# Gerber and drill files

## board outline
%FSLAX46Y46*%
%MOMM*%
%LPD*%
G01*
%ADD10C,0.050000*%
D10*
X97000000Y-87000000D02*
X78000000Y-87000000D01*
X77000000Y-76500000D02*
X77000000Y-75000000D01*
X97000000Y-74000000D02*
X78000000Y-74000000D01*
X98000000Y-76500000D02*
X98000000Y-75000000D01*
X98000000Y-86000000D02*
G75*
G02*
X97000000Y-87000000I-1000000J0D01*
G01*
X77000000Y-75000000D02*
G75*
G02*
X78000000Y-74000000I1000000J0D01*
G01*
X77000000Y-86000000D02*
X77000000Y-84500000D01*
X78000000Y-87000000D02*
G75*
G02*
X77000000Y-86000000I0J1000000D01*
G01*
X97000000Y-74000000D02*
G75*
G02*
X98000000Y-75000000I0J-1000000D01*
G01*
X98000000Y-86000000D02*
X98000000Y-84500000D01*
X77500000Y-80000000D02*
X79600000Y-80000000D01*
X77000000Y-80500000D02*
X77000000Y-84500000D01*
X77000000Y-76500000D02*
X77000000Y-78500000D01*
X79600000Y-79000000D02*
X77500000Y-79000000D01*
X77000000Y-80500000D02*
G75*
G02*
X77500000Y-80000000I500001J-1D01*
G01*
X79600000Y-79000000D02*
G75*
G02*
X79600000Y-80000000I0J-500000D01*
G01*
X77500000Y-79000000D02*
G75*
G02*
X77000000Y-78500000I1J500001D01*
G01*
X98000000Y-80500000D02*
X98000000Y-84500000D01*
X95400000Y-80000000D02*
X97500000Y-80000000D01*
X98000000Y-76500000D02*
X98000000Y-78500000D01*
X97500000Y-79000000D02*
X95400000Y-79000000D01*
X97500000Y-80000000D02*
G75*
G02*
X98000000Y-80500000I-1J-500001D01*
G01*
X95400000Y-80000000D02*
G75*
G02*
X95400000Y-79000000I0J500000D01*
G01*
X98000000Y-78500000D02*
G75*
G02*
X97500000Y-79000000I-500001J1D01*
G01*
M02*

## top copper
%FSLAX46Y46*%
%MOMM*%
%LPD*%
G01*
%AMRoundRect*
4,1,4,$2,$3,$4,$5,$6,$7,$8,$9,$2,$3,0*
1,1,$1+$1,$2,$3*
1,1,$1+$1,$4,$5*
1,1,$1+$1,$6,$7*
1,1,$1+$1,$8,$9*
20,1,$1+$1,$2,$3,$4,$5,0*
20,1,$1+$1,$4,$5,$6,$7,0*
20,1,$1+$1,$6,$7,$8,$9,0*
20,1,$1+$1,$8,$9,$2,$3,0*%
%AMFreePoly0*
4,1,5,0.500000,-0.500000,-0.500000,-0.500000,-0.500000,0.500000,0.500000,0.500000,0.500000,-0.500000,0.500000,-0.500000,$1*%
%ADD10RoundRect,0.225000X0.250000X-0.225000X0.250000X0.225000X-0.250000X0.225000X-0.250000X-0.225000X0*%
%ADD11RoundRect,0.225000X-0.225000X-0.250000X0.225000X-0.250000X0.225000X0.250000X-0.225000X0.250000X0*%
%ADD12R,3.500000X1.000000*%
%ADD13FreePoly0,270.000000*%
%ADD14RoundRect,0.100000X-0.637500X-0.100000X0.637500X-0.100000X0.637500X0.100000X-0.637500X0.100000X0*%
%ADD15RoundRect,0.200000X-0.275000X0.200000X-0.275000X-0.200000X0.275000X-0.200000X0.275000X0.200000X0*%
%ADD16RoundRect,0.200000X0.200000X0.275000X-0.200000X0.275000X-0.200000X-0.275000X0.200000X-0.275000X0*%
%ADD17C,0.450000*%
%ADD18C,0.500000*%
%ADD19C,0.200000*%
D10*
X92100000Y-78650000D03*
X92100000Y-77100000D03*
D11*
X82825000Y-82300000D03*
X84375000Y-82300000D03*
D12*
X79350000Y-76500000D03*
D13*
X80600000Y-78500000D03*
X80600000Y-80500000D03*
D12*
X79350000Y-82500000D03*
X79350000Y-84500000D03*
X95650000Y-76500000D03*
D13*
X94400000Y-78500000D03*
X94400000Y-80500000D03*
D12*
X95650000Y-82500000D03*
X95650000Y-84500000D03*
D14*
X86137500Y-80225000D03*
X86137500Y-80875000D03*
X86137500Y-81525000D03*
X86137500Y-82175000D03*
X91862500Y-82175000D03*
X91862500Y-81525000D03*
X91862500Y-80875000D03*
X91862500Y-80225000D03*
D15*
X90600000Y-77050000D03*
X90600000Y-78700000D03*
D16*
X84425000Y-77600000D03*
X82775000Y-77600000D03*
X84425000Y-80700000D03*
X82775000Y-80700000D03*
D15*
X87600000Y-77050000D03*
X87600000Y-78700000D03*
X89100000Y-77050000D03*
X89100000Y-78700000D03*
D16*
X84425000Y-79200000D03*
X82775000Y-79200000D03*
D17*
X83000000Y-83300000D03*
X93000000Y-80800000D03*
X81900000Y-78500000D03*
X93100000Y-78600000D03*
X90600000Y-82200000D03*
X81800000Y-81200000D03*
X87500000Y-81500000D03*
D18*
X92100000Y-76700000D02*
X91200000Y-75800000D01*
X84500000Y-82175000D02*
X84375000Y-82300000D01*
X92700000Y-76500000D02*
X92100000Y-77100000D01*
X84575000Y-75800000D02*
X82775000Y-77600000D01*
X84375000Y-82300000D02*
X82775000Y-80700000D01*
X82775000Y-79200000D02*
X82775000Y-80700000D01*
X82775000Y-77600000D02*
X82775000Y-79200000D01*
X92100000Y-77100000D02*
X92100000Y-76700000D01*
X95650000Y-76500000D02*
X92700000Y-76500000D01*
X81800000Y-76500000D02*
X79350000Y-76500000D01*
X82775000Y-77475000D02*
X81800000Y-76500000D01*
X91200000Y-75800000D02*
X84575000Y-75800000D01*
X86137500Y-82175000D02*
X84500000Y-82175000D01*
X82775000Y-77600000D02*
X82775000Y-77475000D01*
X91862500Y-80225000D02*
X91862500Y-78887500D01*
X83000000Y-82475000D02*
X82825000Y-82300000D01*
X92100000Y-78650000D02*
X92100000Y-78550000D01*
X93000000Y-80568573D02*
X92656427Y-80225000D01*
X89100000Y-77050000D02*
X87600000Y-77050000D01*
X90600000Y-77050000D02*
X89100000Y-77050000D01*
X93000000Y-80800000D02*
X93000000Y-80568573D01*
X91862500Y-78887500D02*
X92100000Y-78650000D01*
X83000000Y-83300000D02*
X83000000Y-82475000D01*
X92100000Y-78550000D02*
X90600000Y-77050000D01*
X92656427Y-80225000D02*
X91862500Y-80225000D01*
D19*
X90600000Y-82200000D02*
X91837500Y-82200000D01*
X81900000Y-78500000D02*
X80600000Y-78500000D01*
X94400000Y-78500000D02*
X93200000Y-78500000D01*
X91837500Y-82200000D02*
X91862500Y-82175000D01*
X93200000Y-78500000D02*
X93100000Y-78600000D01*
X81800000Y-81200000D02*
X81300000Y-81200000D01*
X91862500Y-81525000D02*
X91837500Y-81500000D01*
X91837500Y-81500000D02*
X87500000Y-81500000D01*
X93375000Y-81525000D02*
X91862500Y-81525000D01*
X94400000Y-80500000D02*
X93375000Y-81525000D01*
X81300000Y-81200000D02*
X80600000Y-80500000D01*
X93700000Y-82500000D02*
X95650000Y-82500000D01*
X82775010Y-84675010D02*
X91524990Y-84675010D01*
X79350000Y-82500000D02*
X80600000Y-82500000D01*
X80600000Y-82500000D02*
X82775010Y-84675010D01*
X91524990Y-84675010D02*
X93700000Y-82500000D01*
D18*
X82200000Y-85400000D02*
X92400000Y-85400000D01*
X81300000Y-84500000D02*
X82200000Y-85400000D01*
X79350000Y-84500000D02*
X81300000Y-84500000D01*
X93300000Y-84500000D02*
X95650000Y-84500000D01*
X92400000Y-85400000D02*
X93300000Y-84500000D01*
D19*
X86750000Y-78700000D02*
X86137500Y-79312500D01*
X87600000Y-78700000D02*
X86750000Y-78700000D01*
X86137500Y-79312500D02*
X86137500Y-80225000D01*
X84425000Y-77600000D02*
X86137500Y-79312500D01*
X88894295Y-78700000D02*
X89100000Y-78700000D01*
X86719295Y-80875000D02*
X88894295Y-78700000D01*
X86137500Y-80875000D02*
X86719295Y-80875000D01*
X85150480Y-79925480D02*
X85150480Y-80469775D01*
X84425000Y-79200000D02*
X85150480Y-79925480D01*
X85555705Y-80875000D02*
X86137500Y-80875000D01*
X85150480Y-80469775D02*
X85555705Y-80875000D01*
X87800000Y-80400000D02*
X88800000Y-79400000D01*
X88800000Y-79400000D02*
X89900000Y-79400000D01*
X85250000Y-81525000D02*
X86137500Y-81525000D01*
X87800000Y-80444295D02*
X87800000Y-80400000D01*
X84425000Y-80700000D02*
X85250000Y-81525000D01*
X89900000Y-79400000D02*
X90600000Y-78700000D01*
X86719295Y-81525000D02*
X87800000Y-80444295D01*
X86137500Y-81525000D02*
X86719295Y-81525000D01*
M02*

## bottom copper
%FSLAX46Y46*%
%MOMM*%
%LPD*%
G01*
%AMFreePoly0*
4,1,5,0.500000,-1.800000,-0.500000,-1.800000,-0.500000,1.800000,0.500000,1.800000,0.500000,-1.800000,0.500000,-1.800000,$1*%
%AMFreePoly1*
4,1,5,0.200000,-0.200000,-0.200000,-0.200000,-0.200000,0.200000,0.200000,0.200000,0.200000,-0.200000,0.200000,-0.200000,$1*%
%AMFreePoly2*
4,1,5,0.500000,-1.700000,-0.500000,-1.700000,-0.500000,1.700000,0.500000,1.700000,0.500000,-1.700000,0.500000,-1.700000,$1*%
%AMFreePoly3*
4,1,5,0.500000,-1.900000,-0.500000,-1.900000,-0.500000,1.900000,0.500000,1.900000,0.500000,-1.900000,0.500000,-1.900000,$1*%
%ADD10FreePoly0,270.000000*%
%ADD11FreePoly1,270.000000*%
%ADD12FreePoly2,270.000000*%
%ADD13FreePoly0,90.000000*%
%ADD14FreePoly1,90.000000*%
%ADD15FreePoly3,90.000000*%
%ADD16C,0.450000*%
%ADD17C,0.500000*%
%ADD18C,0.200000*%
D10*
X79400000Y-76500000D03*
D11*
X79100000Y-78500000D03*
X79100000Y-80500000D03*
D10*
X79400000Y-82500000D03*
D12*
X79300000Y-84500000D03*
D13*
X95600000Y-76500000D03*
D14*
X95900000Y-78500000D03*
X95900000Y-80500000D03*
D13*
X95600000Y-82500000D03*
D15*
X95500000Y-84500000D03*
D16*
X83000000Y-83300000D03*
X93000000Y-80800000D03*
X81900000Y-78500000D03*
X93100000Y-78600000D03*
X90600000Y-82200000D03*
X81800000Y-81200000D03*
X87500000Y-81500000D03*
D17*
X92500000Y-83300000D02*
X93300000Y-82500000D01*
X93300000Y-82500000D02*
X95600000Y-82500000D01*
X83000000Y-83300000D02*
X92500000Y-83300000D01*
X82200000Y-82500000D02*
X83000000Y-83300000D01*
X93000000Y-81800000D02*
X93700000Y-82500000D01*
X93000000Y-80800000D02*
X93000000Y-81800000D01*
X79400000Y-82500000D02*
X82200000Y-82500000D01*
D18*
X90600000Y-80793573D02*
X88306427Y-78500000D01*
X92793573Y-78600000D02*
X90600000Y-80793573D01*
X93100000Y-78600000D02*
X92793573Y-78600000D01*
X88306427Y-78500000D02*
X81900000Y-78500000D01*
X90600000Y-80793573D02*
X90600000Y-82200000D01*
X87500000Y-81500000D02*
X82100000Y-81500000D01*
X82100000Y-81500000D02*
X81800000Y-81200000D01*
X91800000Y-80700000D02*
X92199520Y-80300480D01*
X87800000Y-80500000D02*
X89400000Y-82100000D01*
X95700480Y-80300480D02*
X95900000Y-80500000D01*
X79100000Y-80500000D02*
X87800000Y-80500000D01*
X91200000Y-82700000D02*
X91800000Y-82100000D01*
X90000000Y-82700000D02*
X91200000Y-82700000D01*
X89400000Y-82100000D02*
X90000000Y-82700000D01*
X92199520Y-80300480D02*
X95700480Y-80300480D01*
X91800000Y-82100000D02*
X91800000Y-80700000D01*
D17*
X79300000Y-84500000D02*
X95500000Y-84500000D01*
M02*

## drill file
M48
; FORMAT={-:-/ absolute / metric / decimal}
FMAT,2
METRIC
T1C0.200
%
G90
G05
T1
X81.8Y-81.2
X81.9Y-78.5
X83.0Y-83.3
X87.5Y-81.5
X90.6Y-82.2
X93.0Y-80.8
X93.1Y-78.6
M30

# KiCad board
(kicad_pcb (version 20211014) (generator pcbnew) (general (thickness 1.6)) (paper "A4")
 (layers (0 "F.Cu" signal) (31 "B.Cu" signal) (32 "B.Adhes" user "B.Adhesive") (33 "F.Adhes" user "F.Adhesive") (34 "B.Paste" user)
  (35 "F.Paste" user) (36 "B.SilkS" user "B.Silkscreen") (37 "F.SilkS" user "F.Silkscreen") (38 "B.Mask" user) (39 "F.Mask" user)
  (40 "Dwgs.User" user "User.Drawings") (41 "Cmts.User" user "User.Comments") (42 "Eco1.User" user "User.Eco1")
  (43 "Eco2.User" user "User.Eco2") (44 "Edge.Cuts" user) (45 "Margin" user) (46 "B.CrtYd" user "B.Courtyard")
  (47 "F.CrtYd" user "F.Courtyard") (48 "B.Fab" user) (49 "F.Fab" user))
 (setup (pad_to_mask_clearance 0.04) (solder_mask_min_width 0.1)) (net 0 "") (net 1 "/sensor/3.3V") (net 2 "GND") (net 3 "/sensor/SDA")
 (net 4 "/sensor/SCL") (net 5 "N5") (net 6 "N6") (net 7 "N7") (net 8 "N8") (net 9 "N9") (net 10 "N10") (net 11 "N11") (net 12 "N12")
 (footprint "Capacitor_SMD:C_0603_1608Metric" (layer "F.Cu") (at 92.1 77.875 90)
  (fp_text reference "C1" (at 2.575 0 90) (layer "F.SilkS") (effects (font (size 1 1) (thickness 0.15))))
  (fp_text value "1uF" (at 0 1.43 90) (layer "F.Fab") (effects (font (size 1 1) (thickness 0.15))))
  (pad "1" smd roundrect locked (at -0.775 0 90) (size 0.9 0.95) (layers "F.Cu" "F.Paste" "F.Mask") (roundrect_rratio 0.25)
   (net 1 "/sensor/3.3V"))
  (pad "2" smd roundrect locked (at 0.775 0 90) (size 0.9 0.95) (layers "F.Cu" "F.Paste" "F.Mask") (roundrect_rratio 0.25) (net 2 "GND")))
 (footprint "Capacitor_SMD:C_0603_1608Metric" (layer "F.Cu") (at 83.6 82.3)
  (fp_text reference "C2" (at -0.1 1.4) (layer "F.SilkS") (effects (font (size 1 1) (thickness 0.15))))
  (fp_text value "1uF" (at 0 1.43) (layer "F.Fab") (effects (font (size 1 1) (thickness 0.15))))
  (pad "1" smd roundrect locked (at -0.775 0) (size 0.9 0.95) (layers "F.Cu" "F.Paste" "F.Mask") (roundrect_rratio 0.25)
   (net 1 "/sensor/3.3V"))
  (pad "2" smd roundrect locked (at 0.775 0) (size 0.9 0.95) (layers "F.Cu" "F.Paste" "F.Mask") (roundrect_rratio 0.25) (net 2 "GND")))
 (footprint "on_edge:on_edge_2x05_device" (layer "F.Cu") (at 77 80.5 -90)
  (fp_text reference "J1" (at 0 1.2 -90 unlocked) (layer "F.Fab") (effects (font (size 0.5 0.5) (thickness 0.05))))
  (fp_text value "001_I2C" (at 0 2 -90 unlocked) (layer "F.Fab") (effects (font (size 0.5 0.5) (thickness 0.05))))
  (fp_line (start -0.5 -0.5) (end -0.5 -2.6) (layer "Edge.Cuts") (width 0.05))
  (fp_line (start 0 0) (end 4 0) (layer "Edge.Cuts") (width 0.05))
  (fp_line (start -4 0) (end -2 0) (layer "Edge.Cuts") (width 0.05))
  (fp_line (start -1.5 -2.6) (end -1.5 -0.5) (layer "Edge.Cuts") (width 0.05))
  (fp_arc (start 0 0) (mid -0.353553 -0.146447) (end -0.5 -0.5) (layer "Edge.Cuts") (width 0.05))
  (fp_arc (start -1.5 -2.6) (mid -1 -3.1) (end -0.5 -2.6) (layer "Edge.Cuts") (width 0.05))
  (fp_arc (start -1.5 -0.5) (mid -1.646447 -0.146447) (end -2 0) (layer "Edge.Cuts") (width 0.05))
  (pad "1" smd rect locked (at -4 -2.35 90) (size 1 3.5) (layers "F.Cu" "F.Mask") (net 2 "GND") (zone_connect 0))
  (pad "2" smd custom locked (at -2 -3.6 270) (size 1 1) (layers "F.Cu" "F.Mask") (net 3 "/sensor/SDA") (zone_connect 0)
   (options (clearance outline) (anchor rect)) (primitives))
  (pad "3" smd custom locked (at 0 -3.6 270) (size 1 1) (layers "F.Cu" "F.Mask") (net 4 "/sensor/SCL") (zone_connect 0)
   (options (clearance outline) (anchor rect)) (primitives))
  (pad "4" smd rect locked (at 2 -2.35 90) (size 1 3.5) (layers "F.Cu" "F.Mask") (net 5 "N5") (zone_connect 0))
  (pad "5" smd rect locked (at 4 -2.35 90) (size 1 3.5) (layers "F.Cu" "F.Mask") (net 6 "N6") (zone_connect 0))
  (pad "6" smd custom locked (at -4 -2.4 270) (size 1 3.6) (layers "B.Cu" "B.Mask") (zone_connect 0)
   (options (clearance outline) (anchor rect)) (primitives))
  (pad "7" smd custom locked (at -2 -2.1 270) (size 0.4 0.4) (layers "B.Cu" "B.Mask") (zone_connect 0)
   (options (clearance outline) (anchor rect)) (primitives))
  (pad "8" smd custom locked (at 0 -2.1 270) (size 0.4 0.4) (layers "B.Cu" "B.Mask") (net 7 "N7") (zone_connect 0)
   (options (clearance outline) (anchor rect)) (primitives))
  (pad "9" smd custom locked (at 2 -2.4 270) (size 1 3.6) (layers "B.Cu" "B.Mask") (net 1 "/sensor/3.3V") (zone_connect 0)
   (options (clearance outline) (anchor rect)) (primitives))
  (pad "10" smd custom locked (at 4 -2.3 270) (size 1 3.4) (layers "B.Cu" "B.Mask") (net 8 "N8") (zone_connect 0)
   (options (clearance outline) (anchor rect)) (primitives)))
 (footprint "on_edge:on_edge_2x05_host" (layer "F.Cu") (at 98 80.5 -90)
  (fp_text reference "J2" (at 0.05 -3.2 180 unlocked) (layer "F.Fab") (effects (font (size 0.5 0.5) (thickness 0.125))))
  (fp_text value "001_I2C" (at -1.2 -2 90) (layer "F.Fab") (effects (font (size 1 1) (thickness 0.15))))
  (fp_line (start 0 0) (end 4 0) (layer "Edge.Cuts") (width 0.05))
  (fp_line (start -0.5 2.6) (end -0.5 0.5) (layer "Edge.Cuts") (width 0.05))
  (fp_line (start -4 0) (end -2 0) (layer "Edge.Cuts") (width 0.05))
  (fp_line (start -1.5 0.5) (end -1.5 2.6) (layer "Edge.Cuts") (width 0.05))
  (fp_arc (start -0.5 0.5) (mid -0.353553 0.146447) (end 0 0) (layer "Edge.Cuts") (width 0.05))
  (fp_arc (start -0.5 2.6) (mid -1 3.1) (end -1.5 2.6) (layer "Edge.Cuts") (width 0.05))
  (fp_arc (start -2 0) (mid -1.646447 0.146447) (end -1.5 0.5) (layer "Edge.Cuts") (width 0.05))
  (pad "1" smd rect locked (at -4 2.35 270) (size 1 3.5) (layers "F.Cu" "F.Mask") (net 2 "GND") (zone_connect 0))
  (pad "2" smd custom locked (at -2 3.6 270) (size 1 1) (layers "F.Cu" "F.Mask") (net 3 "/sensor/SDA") (zone_connect 0)
   (options (clearance outline) (anchor rect)) (primitives))
  (pad "3" smd custom locked (at 0 3.6 270) (size 1 1) (layers "F.Cu" "F.Mask") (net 4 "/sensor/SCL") (zone_connect 0)
   (options (clearance outline) (anchor rect)) (primitives))
  (pad "4" smd rect locked (at 2 2.35 270) (size 1 3.5) (layers "F.Cu" "F.Mask") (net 5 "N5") (zone_connect 0))
  (pad "5" smd rect locked (at 4 2.35 270) (size 1 3.5) (layers "F.Cu" "F.Mask") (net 6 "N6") (zone_connect 0))
  (pad "6" smd custom locked (at -4 2.4 90) (size 1 3.6) (layers "B.Cu" "B.Mask") (zone_connect 0)
   (options (clearance outline) (anchor rect)) (primitives))
  (pad "7" smd custom locked (at -2 2.1 90) (size 0.4 0.4) (layers "B.Cu" "B.Mask") (zone_connect 0)
   (options (clearance outline) (anchor rect)) (primitives))
  (pad "8" smd custom locked (at 0 2.1 90) (size 0.4 0.4) (layers "B.Cu" "B.Mask") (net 7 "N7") (zone_connect 0)
   (options (clearance outline) (anchor rect)) (primitives))
  (pad "9" smd custom locked (at 2 2.4 90) (size 1 3.6) (layers "B.Cu" "B.Mask") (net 1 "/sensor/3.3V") (zone_connect 0)
   (options (clearance outline) (anchor rect)) (primitives))
  (pad "10" smd custom locked (at 4 2.5 90) (size 1 3.8) (layers "B.Cu" "B.Mask") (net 8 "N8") (zone_connect 0)
   (options (clearance outline) (anchor rect)) (primitives)))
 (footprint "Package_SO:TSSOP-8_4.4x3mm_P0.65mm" (layer "F.Cu") (at 89 81.2)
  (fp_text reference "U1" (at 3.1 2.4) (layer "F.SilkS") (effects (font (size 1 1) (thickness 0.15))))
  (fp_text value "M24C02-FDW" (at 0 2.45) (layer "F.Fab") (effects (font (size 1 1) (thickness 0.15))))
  (pad "1" smd roundrect locked (at -2.8625 -0.975) (size 1.475 0.4) (layers "F.Cu" "F.Paste" "F.Mask") (roundrect_rratio 0.25) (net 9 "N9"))
  (pad "2" smd roundrect locked (at -2.8625 -0.325) (size 1.475 0.4) (layers "F.Cu" "F.Paste" "F.Mask") (roundrect_rratio 0.25)
   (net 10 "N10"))
  (pad "3" smd roundrect locked (at -2.8625 0.325) (size 1.475 0.4) (layers "F.Cu" "F.Paste" "F.Mask") (roundrect_rratio 0.25)
   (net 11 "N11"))
  (pad "4" smd roundrect locked (at -2.8625 0.975) (size 1.475 0.4) (layers "F.Cu" "F.Paste" "F.Mask") (roundrect_rratio 0.25) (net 2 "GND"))
  (pad "5" smd roundrect locked (at 2.8625 0.975) (size 1.475 0.4) (layers "F.Cu" "F.Paste" "F.Mask") (roundrect_rratio 0.25)
   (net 3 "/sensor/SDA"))
  (pad "6" smd roundrect locked (at 2.8625 0.325) (size 1.475 0.4) (layers "F.Cu" "F.Paste" "F.Mask") (roundrect_rratio 0.25)
   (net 4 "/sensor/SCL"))
  (pad "7" smd roundrect locked (at 2.8625 -0.325) (size 1.475 0.4) (layers "F.Cu" "F.Paste" "F.Mask") (roundrect_rratio 0.25)
   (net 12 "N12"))
  (pad "8" smd roundrect locked (at 2.8625 -0.975) (size 1.475 0.4) (layers "F.Cu" "F.Paste" "F.Mask") (roundrect_rratio 0.25)
   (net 1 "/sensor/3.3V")))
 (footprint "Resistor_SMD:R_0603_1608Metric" (layer "F.Cu") (at 90.6 77.875 -90)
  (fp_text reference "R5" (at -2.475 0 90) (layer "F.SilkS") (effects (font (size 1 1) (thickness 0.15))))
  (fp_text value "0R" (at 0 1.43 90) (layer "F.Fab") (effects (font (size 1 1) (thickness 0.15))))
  (pad "1" smd roundrect locked (at -0.825 0 270) (size 0.8 0.95) (layers "F.Cu" "F.Paste" "F.Mask") (roundrect_rratio 0.25)
   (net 1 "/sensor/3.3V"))
  (pad "2" smd roundrect locked (at 0.825 0 270) (size 0.8 0.95) (layers "F.Cu" "F.Paste" "F.Mask") (roundrect_rratio 0.25) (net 11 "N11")))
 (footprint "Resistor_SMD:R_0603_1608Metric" (layer "F.Cu") (at 83.6 77.6 180)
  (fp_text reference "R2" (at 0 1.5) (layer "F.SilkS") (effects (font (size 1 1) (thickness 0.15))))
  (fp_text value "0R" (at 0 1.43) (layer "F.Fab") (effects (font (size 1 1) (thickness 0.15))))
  (pad "1" smd roundrect locked (at -0.825 0 180) (size 0.8 0.95) (layers "F.Cu" "F.Paste" "F.Mask") (roundrect_rratio 0.25) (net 9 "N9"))
  (pad "2" smd roundrect locked (at 0.825 0 180) (size 0.8 0.95) (layers "F.Cu" "F.Paste" "F.Mask") (roundrect_rratio 0.25) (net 2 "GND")))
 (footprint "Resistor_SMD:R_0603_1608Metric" (layer "F.Cu") (at 83.6 80.7 180)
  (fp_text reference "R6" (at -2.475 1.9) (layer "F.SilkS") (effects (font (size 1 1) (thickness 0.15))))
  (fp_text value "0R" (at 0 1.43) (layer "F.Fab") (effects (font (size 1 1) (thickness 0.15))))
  (pad "1" smd roundrect locked (at -0.825 0 180) (size 0.8 0.95) (layers "F.Cu" "F.Paste" "F.Mask") (roundrect_rratio 0.25) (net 11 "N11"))
  (pad "2" smd roundrect locked (at 0.825 0 180) (size 0.8 0.95) (layers "F.Cu" "F.Paste" "F.Mask") (roundrect_rratio 0.25) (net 2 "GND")))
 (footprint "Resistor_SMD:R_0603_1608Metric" (layer "F.Cu") (at 87.6 77.875 -90)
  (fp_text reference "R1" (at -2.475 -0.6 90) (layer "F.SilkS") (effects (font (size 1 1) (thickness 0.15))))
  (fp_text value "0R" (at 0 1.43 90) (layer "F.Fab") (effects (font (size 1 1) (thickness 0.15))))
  (pad "1" smd roundrect locked (at -0.825 0 270) (size 0.8 0.95) (layers "F.Cu" "F.Paste" "F.Mask") (roundrect_rratio 0.25)
   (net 1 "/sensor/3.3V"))
  (pad "2" smd roundrect locked (at 0.825 0 270) (size 0.8 0.95) (layers "F.Cu" "F.Paste" "F.Mask") (roundrect_rratio 0.25) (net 9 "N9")))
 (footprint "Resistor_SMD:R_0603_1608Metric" (layer "F.Cu") (at 89.1 77.875 -90)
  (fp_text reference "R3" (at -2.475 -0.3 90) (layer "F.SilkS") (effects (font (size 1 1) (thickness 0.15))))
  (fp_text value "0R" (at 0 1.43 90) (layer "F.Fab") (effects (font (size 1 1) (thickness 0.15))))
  (pad "1" smd roundrect locked (at -0.825 0 270) (size 0.8 0.95) (layers "F.Cu" "F.Paste" "F.Mask") (roundrect_rratio 0.25)
   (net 1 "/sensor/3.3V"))
  (pad "2" smd roundrect locked (at 0.825 0 270) (size 0.8 0.95) (layers "F.Cu" "F.Paste" "F.Mask") (roundrect_rratio 0.25) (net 10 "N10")))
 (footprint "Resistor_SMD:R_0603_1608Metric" (layer "F.Cu") (at 83.6 79.2 180)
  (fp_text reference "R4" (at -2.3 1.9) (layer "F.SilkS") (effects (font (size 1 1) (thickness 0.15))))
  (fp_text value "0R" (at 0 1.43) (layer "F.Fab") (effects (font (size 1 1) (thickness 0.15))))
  (pad "1" smd roundrect locked (at -0.825 0 180) (size 0.8 0.95) (layers "F.Cu" "F.Paste" "F.Mask") (roundrect_rratio 0.25) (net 10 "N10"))
  (pad "2" smd roundrect locked (at 0.825 0 180) (size 0.8 0.95) (layers "F.Cu" "F.Paste" "F.Mask") (roundrect_rratio 0.25) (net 2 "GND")))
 (gr_line (start 97 87) (end 78 87) (layer "Edge.Cuts") (width 0.05))
 (gr_line (start 77 76.5) (end 77 75) (layer "Edge.Cuts") (width 0.05))
 (gr_line (start 97 74) (end 78 74) (layer "Edge.Cuts") (width 0.05))
 (gr_line (start 98 76.5) (end 98 75) (layer "Edge.Cuts") (width 0.05))
 (gr_arc (start 98 86) (mid 97.707107 86.707107) (end 97 87) (layer "Edge.Cuts") (width 0.05))
 (gr_arc (start 77 75) (mid 77.292893 74.292893) (end 78 74) (layer "Edge.Cuts") (width 0.05))
 (gr_line (start 77 86) (end 77 84.5) (layer "Edge.Cuts") (width 0.05))
 (gr_arc (start 78 87) (mid 77.292893 86.707107) (end 77 86) (layer "Edge.Cuts") (width 0.05))
 (gr_arc (start 97 74) (mid 97.707107 74.292893) (end 98 75) (layer "Edge.Cuts") (width 0.05))
 (gr_line (start 98 86) (end 98 84.5) (layer "Edge.Cuts") (width 0.05))
 (segment (start 92.1 76.7) (end 91.2 75.8) (width 0.5) (layer "F.Cu") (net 2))
 (segment (start 84.5 82.175) (end 84.375 82.3) (width 0.5) (layer "F.Cu") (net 2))
 (segment (start 92.7 76.5) (end 92.1 77.1) (width 0.5) (layer "F.Cu") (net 2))
 (segment (start 84.575 75.8) (end 82.775 77.6) (width 0.5) (layer "F.Cu") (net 2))
 (segment (start 84.375 82.3) (end 82.775 80.7) (width 0.5) (layer "F.Cu") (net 2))
 (segment (start 82.775 79.2) (end 82.775 80.7) (width 0.5) (layer "F.Cu") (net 2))
 (segment (start 82.775 77.6) (end 82.775 79.2) (width 0.5) (layer "F.Cu") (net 2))
 (segment (start 92.1 77.1) (end 92.1 76.7) (width 0.5) (layer "F.Cu") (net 2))
 (segment (start 95.65 76.5) (end 92.7 76.5) (width 0.5) (layer "F.Cu") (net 2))
 (segment (start 81.8 76.5) (end 79.35 76.5) (width 0.5) (layer "F.Cu") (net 2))
 (segment (start 82.775 77.475) (end 81.8 76.5) (width 0.5) (layer "F.Cu") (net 2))
 (segment (start 91.2 75.8) (end 84.575 75.8) (width 0.5) (layer "F.Cu") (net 2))
 (segment (start 86.1375 82.175) (end 84.5 82.175) (width 0.5) (layer "F.Cu") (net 2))
 (segment (start 82.775 77.6) (end 82.775 77.475) (width 0.5) (layer "F.Cu") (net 2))
 (segment (start 91.8625 80.225) (end 91.8625 78.8875) (width 0.5) (layer "F.Cu") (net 1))
 (segment (start 83 82.475) (end 82.825 82.3) (width 0.5) (layer "F.Cu") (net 1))
 (segment (start 92.1 78.65) (end 92.1 78.55) (width 0.5) (layer "F.Cu") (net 1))
 (segment (start 93 80.568573) (end 92.656427 80.225) (width 0.5) (layer "F.Cu") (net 1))
 (segment (start 89.1 77.05) (end 87.6 77.05) (width 0.5) (layer "F.Cu") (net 1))
 (segment (start 90.6 77.05) (end 89.1 77.05) (width 0.5) (layer "F.Cu") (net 1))
 (segment (start 93 80.8) (end 93 80.568573) (width 0.5) (layer "F.Cu") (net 1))
 (segment (start 91.8625 78.8875) (end 92.1 78.65) (width 0.5) (layer "F.Cu") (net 1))
 (segment (start 83 83.3) (end 83 82.475) (width 0.5) (layer "F.Cu") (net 1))
 (segment (start 92.1 78.55) (end 90.6 77.05) (width 0.5) (layer "F.Cu") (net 1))
 (segment (start 92.656427 80.225) (end 91.8625 80.225) (width 0.5) (layer "F.Cu") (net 1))
 (via (at 83 83.3) (size 0.45) (drill 0.2) (layers "F.Cu" "B.Cu") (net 1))
 (via (at 93 80.8) (size 0.45) (drill 0.2) (layers "F.Cu" "B.Cu") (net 1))
 (segment (start 92.5 83.3) (end 93.3 82.5) (width 0.5) (layer "B.Cu") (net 1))
 (segment (start 93.3 82.5) (end 95.6 82.5) (width 0.5) (layer "B.Cu") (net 1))
 (segment (start 83 83.3) (end 92.5 83.3) (width 0.5) (layer "B.Cu") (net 1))
 (segment (start 82.2 82.5) (end 83 83.3) (width 0.5) (layer "B.Cu") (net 1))
 (segment (start 93 81.8) (end 93.7 82.5) (width 0.5) (layer "B.Cu") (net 1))
 (segment (start 93 80.8) (end 93 81.8) (width 0.5) (layer "B.Cu") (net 1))
 (segment (start 79.4 82.5) (end 82.2 82.5) (width 0.5) (layer "B.Cu") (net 1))
 (segment (start 90.6 82.2) (end 91.8375 82.2) (width 0.2) (layer "F.Cu") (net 3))
 (segment (start 81.9 78.5) (end 80.6 78.5) (width 0.2) (layer "F.Cu") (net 3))
 (segment (start 94.4 78.5) (end 93.2 78.5) (width 0.2) (layer "F.Cu") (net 3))
 (segment (start 91.8375 82.2) (end 91.8625 82.175) (width 0.2) (layer "F.Cu") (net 3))
 (segment (start 93.2 78.5) (end 93.1 78.6) (width 0.2) (layer "F.Cu") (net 3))
 (via (at 81.9 78.5) (size 0.45) (drill 0.2) (layers "F.Cu" "B.Cu") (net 3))
 (via (at 93.1 78.6) (size 0.45) (drill 0.2) (layers "F.Cu" "B.Cu") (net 3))
 (via (at 90.6 82.2) (size 0.45) (drill 0.2) (layers "F.Cu" "B.Cu") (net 3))
 (segment (start 90.6 80.793573) (end 88.306427 78.5) (width 0.2) (layer "B.Cu") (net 3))
 (segment (start 92.793573 78.6) (end 90.6 80.793573) (width 0.2) (layer "B.Cu") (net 3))
 (segment (start 93.1 78.6) (end 92.793573 78.6) (width 0.2) (layer "B.Cu") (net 3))
 (segment (start 88.306427 78.5) (end 81.9 78.5) (width 0.2) (layer "B.Cu") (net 3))
 (segment (start 90.6 80.793573) (end 90.6 82.2) (width 0.2) (layer "B.Cu") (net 3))
 (segment (start 81.8 81.2) (end 81.3 81.2) (width 0.2) (layer "F.Cu") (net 4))
 (segment (start 91.8625 81.525) (end 91.8375 81.5) (width 0.2) (layer "F.Cu") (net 4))
 (segment (start 91.8375 81.5) (end 87.5 81.5) (width 0.2) (layer "F.Cu") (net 4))
 (segment (start 93.375 81.525) (end 91.8625 81.525) (width 0.2) (layer "F.Cu") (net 4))
 (segment (start 94.4 80.5) (end 93.375 81.525) (width 0.2) (layer "F.Cu") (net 4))
 (segment (start 81.3 81.2) (end 80.6 80.5) (width 0.2) (layer "F.Cu") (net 4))
 (via (at 81.8 81.2) (size 0.45) (drill 0.2) (layers "F.Cu" "B.Cu") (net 4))
 (via (at 87.5 81.5) (size 0.45) (drill 0.2) (layers "F.Cu" "B.Cu") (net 4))
 (segment (start 87.5 81.5) (end 82.1 81.5) (width 0.2) (layer "B.Cu") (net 4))
 (segment (start 82.1 81.5) (end 81.8 81.2) (width 0.2) (layer "B.Cu") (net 4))
 (segment (start 91.8 80.7) (end 92.19952 80.30048) (width 0.2) (layer "B.Cu") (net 7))
 (segment (start 87.8 80.5) (end 89.4 82.1) (width 0.2) (layer "B.Cu") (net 7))
 (segment (start 95.70048 80.30048) (end 95.9 80.5) (width 0.2) (layer "B.Cu") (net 7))
 (segment (start 79.1 80.5) (end 87.8 80.5) (width 0.2) (layer "B.Cu") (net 7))
 (segment (start 91.2 82.7) (end 91.8 82.1) (width 0.2) (layer "B.Cu") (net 7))
 (segment (start 90 82.7) (end 91.2 82.7) (width 0.2) (layer "B.Cu") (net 7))
 (segment (start 89.4 82.1) (end 90 82.7) (width 0.2) (layer "B.Cu") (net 7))
 (segment (start 92.19952 80.30048) (end 95.70048 80.30048) (width 0.2) (layer "B.Cu") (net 7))
 (segment (start 91.8 82.1) (end 91.8 80.7) (width 0.2) (layer "B.Cu") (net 7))
 (segment (start 79.3 84.5) (end 95.5 84.5) (width 0.5) (layer "B.Cu") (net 8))
 (segment (start 93.7 82.5) (end 95.65 82.5) (width 0.2) (layer "F.Cu") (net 5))
 (segment (start 82.77501 84.67501) (end 91.52499 84.67501) (width 0.2) (layer "F.Cu") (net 5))
 (segment (start 79.35 82.5) (end 80.6 82.5) (width 0.2) (layer "F.Cu") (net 5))
 (segment (start 80.6 82.5) (end 82.77501 84.67501) (width 0.2) (layer "F.Cu") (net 5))
 (segment (start 91.52499 84.67501) (end 93.7 82.5) (width 0.2) (layer "F.Cu") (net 5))
 (segment (start 82.2 85.4) (end 92.4 85.4) (width 0.5) (layer "F.Cu") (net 6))
 (segment (start 81.3 84.5) (end 82.2 85.4) (width 0.5) (layer "F.Cu") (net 6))
 (segment (start 79.35 84.5) (end 81.3 84.5) (width 0.5) (layer "F.Cu") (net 6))
 (segment (start 93.3 84.5) (end 95.65 84.5) (width 0.5) (layer "F.Cu") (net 6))
 (segment (start 92.4 85.4) (end 93.3 84.5) (width 0.5) (layer "F.Cu") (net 6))
 (segment (start 86.75 78.7) (end 86.1375 79.3125) (width 0.2) (layer "F.Cu") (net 9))
 (segment (start 87.6 78.7) (end 86.75 78.7) (width 0.2) (layer "F.Cu") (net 9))
 (segment (start 86.1375 79.3125) (end 86.1375 80.225) (width 0.2) (layer "F.Cu") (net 9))
 (segment (start 84.425 77.6) (end 86.1375 79.3125) (width 0.2) (layer "F.Cu") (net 9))
 (segment (start 88.894295 78.7) (end 89.1 78.7) (width 0.2) (layer "F.Cu") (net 10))
 (segment (start 86.719295 80.875) (end 88.894295 78.7) (width 0.2) (layer "F.Cu") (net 10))
 (segment (start 86.1375 80.875) (end 86.719295 80.875) (width 0.2) (layer "F.Cu") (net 10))
 (segment (start 85.15048 79.92548) (end 85.15048 80.469775) (width 0.2) (layer "F.Cu") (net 10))
 (segment (start 84.425 79.2) (end 85.15048 79.92548) (width 0.2) (layer "F.Cu") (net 10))
 (segment (start 85.555705 80.875) (end 86.1375 80.875) (width 0.2) (layer "F.Cu") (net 10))
 (segment (start 85.15048 80.469775) (end 85.555705 80.875) (width 0.2) (layer "F.Cu") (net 10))
 (segment (start 87.8 80.4) (end 88.8 79.4) (width 0.2) (layer "F.Cu") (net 11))
 (segment (start 88.8 79.4) (end 89.9 79.4) (width 0.2) (layer "F.Cu") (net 11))
 (segment (start 85.25 81.525) (end 86.1375 81.525) (width 0.2) (layer "F.Cu") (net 11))
 (segment (start 87.8 80.444295) (end 87.8 80.4) (width 0.2) (layer "F.Cu") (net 11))
 (segment (start 84.425 80.7) (end 85.25 81.525) (width 0.2) (layer "F.Cu") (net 11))
 (segment (start 89.9 79.4) (end 90.6 78.7) (width 0.2) (layer "F.Cu") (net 11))
 (segment (start 86.719295 81.525) (end 87.8 80.444295) (width 0.2) (layer "F.Cu") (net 11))
 (segment (start 86.1375 81.525) (end 86.719295 81.525) (width 0.2) (layer "F.Cu") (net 11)))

